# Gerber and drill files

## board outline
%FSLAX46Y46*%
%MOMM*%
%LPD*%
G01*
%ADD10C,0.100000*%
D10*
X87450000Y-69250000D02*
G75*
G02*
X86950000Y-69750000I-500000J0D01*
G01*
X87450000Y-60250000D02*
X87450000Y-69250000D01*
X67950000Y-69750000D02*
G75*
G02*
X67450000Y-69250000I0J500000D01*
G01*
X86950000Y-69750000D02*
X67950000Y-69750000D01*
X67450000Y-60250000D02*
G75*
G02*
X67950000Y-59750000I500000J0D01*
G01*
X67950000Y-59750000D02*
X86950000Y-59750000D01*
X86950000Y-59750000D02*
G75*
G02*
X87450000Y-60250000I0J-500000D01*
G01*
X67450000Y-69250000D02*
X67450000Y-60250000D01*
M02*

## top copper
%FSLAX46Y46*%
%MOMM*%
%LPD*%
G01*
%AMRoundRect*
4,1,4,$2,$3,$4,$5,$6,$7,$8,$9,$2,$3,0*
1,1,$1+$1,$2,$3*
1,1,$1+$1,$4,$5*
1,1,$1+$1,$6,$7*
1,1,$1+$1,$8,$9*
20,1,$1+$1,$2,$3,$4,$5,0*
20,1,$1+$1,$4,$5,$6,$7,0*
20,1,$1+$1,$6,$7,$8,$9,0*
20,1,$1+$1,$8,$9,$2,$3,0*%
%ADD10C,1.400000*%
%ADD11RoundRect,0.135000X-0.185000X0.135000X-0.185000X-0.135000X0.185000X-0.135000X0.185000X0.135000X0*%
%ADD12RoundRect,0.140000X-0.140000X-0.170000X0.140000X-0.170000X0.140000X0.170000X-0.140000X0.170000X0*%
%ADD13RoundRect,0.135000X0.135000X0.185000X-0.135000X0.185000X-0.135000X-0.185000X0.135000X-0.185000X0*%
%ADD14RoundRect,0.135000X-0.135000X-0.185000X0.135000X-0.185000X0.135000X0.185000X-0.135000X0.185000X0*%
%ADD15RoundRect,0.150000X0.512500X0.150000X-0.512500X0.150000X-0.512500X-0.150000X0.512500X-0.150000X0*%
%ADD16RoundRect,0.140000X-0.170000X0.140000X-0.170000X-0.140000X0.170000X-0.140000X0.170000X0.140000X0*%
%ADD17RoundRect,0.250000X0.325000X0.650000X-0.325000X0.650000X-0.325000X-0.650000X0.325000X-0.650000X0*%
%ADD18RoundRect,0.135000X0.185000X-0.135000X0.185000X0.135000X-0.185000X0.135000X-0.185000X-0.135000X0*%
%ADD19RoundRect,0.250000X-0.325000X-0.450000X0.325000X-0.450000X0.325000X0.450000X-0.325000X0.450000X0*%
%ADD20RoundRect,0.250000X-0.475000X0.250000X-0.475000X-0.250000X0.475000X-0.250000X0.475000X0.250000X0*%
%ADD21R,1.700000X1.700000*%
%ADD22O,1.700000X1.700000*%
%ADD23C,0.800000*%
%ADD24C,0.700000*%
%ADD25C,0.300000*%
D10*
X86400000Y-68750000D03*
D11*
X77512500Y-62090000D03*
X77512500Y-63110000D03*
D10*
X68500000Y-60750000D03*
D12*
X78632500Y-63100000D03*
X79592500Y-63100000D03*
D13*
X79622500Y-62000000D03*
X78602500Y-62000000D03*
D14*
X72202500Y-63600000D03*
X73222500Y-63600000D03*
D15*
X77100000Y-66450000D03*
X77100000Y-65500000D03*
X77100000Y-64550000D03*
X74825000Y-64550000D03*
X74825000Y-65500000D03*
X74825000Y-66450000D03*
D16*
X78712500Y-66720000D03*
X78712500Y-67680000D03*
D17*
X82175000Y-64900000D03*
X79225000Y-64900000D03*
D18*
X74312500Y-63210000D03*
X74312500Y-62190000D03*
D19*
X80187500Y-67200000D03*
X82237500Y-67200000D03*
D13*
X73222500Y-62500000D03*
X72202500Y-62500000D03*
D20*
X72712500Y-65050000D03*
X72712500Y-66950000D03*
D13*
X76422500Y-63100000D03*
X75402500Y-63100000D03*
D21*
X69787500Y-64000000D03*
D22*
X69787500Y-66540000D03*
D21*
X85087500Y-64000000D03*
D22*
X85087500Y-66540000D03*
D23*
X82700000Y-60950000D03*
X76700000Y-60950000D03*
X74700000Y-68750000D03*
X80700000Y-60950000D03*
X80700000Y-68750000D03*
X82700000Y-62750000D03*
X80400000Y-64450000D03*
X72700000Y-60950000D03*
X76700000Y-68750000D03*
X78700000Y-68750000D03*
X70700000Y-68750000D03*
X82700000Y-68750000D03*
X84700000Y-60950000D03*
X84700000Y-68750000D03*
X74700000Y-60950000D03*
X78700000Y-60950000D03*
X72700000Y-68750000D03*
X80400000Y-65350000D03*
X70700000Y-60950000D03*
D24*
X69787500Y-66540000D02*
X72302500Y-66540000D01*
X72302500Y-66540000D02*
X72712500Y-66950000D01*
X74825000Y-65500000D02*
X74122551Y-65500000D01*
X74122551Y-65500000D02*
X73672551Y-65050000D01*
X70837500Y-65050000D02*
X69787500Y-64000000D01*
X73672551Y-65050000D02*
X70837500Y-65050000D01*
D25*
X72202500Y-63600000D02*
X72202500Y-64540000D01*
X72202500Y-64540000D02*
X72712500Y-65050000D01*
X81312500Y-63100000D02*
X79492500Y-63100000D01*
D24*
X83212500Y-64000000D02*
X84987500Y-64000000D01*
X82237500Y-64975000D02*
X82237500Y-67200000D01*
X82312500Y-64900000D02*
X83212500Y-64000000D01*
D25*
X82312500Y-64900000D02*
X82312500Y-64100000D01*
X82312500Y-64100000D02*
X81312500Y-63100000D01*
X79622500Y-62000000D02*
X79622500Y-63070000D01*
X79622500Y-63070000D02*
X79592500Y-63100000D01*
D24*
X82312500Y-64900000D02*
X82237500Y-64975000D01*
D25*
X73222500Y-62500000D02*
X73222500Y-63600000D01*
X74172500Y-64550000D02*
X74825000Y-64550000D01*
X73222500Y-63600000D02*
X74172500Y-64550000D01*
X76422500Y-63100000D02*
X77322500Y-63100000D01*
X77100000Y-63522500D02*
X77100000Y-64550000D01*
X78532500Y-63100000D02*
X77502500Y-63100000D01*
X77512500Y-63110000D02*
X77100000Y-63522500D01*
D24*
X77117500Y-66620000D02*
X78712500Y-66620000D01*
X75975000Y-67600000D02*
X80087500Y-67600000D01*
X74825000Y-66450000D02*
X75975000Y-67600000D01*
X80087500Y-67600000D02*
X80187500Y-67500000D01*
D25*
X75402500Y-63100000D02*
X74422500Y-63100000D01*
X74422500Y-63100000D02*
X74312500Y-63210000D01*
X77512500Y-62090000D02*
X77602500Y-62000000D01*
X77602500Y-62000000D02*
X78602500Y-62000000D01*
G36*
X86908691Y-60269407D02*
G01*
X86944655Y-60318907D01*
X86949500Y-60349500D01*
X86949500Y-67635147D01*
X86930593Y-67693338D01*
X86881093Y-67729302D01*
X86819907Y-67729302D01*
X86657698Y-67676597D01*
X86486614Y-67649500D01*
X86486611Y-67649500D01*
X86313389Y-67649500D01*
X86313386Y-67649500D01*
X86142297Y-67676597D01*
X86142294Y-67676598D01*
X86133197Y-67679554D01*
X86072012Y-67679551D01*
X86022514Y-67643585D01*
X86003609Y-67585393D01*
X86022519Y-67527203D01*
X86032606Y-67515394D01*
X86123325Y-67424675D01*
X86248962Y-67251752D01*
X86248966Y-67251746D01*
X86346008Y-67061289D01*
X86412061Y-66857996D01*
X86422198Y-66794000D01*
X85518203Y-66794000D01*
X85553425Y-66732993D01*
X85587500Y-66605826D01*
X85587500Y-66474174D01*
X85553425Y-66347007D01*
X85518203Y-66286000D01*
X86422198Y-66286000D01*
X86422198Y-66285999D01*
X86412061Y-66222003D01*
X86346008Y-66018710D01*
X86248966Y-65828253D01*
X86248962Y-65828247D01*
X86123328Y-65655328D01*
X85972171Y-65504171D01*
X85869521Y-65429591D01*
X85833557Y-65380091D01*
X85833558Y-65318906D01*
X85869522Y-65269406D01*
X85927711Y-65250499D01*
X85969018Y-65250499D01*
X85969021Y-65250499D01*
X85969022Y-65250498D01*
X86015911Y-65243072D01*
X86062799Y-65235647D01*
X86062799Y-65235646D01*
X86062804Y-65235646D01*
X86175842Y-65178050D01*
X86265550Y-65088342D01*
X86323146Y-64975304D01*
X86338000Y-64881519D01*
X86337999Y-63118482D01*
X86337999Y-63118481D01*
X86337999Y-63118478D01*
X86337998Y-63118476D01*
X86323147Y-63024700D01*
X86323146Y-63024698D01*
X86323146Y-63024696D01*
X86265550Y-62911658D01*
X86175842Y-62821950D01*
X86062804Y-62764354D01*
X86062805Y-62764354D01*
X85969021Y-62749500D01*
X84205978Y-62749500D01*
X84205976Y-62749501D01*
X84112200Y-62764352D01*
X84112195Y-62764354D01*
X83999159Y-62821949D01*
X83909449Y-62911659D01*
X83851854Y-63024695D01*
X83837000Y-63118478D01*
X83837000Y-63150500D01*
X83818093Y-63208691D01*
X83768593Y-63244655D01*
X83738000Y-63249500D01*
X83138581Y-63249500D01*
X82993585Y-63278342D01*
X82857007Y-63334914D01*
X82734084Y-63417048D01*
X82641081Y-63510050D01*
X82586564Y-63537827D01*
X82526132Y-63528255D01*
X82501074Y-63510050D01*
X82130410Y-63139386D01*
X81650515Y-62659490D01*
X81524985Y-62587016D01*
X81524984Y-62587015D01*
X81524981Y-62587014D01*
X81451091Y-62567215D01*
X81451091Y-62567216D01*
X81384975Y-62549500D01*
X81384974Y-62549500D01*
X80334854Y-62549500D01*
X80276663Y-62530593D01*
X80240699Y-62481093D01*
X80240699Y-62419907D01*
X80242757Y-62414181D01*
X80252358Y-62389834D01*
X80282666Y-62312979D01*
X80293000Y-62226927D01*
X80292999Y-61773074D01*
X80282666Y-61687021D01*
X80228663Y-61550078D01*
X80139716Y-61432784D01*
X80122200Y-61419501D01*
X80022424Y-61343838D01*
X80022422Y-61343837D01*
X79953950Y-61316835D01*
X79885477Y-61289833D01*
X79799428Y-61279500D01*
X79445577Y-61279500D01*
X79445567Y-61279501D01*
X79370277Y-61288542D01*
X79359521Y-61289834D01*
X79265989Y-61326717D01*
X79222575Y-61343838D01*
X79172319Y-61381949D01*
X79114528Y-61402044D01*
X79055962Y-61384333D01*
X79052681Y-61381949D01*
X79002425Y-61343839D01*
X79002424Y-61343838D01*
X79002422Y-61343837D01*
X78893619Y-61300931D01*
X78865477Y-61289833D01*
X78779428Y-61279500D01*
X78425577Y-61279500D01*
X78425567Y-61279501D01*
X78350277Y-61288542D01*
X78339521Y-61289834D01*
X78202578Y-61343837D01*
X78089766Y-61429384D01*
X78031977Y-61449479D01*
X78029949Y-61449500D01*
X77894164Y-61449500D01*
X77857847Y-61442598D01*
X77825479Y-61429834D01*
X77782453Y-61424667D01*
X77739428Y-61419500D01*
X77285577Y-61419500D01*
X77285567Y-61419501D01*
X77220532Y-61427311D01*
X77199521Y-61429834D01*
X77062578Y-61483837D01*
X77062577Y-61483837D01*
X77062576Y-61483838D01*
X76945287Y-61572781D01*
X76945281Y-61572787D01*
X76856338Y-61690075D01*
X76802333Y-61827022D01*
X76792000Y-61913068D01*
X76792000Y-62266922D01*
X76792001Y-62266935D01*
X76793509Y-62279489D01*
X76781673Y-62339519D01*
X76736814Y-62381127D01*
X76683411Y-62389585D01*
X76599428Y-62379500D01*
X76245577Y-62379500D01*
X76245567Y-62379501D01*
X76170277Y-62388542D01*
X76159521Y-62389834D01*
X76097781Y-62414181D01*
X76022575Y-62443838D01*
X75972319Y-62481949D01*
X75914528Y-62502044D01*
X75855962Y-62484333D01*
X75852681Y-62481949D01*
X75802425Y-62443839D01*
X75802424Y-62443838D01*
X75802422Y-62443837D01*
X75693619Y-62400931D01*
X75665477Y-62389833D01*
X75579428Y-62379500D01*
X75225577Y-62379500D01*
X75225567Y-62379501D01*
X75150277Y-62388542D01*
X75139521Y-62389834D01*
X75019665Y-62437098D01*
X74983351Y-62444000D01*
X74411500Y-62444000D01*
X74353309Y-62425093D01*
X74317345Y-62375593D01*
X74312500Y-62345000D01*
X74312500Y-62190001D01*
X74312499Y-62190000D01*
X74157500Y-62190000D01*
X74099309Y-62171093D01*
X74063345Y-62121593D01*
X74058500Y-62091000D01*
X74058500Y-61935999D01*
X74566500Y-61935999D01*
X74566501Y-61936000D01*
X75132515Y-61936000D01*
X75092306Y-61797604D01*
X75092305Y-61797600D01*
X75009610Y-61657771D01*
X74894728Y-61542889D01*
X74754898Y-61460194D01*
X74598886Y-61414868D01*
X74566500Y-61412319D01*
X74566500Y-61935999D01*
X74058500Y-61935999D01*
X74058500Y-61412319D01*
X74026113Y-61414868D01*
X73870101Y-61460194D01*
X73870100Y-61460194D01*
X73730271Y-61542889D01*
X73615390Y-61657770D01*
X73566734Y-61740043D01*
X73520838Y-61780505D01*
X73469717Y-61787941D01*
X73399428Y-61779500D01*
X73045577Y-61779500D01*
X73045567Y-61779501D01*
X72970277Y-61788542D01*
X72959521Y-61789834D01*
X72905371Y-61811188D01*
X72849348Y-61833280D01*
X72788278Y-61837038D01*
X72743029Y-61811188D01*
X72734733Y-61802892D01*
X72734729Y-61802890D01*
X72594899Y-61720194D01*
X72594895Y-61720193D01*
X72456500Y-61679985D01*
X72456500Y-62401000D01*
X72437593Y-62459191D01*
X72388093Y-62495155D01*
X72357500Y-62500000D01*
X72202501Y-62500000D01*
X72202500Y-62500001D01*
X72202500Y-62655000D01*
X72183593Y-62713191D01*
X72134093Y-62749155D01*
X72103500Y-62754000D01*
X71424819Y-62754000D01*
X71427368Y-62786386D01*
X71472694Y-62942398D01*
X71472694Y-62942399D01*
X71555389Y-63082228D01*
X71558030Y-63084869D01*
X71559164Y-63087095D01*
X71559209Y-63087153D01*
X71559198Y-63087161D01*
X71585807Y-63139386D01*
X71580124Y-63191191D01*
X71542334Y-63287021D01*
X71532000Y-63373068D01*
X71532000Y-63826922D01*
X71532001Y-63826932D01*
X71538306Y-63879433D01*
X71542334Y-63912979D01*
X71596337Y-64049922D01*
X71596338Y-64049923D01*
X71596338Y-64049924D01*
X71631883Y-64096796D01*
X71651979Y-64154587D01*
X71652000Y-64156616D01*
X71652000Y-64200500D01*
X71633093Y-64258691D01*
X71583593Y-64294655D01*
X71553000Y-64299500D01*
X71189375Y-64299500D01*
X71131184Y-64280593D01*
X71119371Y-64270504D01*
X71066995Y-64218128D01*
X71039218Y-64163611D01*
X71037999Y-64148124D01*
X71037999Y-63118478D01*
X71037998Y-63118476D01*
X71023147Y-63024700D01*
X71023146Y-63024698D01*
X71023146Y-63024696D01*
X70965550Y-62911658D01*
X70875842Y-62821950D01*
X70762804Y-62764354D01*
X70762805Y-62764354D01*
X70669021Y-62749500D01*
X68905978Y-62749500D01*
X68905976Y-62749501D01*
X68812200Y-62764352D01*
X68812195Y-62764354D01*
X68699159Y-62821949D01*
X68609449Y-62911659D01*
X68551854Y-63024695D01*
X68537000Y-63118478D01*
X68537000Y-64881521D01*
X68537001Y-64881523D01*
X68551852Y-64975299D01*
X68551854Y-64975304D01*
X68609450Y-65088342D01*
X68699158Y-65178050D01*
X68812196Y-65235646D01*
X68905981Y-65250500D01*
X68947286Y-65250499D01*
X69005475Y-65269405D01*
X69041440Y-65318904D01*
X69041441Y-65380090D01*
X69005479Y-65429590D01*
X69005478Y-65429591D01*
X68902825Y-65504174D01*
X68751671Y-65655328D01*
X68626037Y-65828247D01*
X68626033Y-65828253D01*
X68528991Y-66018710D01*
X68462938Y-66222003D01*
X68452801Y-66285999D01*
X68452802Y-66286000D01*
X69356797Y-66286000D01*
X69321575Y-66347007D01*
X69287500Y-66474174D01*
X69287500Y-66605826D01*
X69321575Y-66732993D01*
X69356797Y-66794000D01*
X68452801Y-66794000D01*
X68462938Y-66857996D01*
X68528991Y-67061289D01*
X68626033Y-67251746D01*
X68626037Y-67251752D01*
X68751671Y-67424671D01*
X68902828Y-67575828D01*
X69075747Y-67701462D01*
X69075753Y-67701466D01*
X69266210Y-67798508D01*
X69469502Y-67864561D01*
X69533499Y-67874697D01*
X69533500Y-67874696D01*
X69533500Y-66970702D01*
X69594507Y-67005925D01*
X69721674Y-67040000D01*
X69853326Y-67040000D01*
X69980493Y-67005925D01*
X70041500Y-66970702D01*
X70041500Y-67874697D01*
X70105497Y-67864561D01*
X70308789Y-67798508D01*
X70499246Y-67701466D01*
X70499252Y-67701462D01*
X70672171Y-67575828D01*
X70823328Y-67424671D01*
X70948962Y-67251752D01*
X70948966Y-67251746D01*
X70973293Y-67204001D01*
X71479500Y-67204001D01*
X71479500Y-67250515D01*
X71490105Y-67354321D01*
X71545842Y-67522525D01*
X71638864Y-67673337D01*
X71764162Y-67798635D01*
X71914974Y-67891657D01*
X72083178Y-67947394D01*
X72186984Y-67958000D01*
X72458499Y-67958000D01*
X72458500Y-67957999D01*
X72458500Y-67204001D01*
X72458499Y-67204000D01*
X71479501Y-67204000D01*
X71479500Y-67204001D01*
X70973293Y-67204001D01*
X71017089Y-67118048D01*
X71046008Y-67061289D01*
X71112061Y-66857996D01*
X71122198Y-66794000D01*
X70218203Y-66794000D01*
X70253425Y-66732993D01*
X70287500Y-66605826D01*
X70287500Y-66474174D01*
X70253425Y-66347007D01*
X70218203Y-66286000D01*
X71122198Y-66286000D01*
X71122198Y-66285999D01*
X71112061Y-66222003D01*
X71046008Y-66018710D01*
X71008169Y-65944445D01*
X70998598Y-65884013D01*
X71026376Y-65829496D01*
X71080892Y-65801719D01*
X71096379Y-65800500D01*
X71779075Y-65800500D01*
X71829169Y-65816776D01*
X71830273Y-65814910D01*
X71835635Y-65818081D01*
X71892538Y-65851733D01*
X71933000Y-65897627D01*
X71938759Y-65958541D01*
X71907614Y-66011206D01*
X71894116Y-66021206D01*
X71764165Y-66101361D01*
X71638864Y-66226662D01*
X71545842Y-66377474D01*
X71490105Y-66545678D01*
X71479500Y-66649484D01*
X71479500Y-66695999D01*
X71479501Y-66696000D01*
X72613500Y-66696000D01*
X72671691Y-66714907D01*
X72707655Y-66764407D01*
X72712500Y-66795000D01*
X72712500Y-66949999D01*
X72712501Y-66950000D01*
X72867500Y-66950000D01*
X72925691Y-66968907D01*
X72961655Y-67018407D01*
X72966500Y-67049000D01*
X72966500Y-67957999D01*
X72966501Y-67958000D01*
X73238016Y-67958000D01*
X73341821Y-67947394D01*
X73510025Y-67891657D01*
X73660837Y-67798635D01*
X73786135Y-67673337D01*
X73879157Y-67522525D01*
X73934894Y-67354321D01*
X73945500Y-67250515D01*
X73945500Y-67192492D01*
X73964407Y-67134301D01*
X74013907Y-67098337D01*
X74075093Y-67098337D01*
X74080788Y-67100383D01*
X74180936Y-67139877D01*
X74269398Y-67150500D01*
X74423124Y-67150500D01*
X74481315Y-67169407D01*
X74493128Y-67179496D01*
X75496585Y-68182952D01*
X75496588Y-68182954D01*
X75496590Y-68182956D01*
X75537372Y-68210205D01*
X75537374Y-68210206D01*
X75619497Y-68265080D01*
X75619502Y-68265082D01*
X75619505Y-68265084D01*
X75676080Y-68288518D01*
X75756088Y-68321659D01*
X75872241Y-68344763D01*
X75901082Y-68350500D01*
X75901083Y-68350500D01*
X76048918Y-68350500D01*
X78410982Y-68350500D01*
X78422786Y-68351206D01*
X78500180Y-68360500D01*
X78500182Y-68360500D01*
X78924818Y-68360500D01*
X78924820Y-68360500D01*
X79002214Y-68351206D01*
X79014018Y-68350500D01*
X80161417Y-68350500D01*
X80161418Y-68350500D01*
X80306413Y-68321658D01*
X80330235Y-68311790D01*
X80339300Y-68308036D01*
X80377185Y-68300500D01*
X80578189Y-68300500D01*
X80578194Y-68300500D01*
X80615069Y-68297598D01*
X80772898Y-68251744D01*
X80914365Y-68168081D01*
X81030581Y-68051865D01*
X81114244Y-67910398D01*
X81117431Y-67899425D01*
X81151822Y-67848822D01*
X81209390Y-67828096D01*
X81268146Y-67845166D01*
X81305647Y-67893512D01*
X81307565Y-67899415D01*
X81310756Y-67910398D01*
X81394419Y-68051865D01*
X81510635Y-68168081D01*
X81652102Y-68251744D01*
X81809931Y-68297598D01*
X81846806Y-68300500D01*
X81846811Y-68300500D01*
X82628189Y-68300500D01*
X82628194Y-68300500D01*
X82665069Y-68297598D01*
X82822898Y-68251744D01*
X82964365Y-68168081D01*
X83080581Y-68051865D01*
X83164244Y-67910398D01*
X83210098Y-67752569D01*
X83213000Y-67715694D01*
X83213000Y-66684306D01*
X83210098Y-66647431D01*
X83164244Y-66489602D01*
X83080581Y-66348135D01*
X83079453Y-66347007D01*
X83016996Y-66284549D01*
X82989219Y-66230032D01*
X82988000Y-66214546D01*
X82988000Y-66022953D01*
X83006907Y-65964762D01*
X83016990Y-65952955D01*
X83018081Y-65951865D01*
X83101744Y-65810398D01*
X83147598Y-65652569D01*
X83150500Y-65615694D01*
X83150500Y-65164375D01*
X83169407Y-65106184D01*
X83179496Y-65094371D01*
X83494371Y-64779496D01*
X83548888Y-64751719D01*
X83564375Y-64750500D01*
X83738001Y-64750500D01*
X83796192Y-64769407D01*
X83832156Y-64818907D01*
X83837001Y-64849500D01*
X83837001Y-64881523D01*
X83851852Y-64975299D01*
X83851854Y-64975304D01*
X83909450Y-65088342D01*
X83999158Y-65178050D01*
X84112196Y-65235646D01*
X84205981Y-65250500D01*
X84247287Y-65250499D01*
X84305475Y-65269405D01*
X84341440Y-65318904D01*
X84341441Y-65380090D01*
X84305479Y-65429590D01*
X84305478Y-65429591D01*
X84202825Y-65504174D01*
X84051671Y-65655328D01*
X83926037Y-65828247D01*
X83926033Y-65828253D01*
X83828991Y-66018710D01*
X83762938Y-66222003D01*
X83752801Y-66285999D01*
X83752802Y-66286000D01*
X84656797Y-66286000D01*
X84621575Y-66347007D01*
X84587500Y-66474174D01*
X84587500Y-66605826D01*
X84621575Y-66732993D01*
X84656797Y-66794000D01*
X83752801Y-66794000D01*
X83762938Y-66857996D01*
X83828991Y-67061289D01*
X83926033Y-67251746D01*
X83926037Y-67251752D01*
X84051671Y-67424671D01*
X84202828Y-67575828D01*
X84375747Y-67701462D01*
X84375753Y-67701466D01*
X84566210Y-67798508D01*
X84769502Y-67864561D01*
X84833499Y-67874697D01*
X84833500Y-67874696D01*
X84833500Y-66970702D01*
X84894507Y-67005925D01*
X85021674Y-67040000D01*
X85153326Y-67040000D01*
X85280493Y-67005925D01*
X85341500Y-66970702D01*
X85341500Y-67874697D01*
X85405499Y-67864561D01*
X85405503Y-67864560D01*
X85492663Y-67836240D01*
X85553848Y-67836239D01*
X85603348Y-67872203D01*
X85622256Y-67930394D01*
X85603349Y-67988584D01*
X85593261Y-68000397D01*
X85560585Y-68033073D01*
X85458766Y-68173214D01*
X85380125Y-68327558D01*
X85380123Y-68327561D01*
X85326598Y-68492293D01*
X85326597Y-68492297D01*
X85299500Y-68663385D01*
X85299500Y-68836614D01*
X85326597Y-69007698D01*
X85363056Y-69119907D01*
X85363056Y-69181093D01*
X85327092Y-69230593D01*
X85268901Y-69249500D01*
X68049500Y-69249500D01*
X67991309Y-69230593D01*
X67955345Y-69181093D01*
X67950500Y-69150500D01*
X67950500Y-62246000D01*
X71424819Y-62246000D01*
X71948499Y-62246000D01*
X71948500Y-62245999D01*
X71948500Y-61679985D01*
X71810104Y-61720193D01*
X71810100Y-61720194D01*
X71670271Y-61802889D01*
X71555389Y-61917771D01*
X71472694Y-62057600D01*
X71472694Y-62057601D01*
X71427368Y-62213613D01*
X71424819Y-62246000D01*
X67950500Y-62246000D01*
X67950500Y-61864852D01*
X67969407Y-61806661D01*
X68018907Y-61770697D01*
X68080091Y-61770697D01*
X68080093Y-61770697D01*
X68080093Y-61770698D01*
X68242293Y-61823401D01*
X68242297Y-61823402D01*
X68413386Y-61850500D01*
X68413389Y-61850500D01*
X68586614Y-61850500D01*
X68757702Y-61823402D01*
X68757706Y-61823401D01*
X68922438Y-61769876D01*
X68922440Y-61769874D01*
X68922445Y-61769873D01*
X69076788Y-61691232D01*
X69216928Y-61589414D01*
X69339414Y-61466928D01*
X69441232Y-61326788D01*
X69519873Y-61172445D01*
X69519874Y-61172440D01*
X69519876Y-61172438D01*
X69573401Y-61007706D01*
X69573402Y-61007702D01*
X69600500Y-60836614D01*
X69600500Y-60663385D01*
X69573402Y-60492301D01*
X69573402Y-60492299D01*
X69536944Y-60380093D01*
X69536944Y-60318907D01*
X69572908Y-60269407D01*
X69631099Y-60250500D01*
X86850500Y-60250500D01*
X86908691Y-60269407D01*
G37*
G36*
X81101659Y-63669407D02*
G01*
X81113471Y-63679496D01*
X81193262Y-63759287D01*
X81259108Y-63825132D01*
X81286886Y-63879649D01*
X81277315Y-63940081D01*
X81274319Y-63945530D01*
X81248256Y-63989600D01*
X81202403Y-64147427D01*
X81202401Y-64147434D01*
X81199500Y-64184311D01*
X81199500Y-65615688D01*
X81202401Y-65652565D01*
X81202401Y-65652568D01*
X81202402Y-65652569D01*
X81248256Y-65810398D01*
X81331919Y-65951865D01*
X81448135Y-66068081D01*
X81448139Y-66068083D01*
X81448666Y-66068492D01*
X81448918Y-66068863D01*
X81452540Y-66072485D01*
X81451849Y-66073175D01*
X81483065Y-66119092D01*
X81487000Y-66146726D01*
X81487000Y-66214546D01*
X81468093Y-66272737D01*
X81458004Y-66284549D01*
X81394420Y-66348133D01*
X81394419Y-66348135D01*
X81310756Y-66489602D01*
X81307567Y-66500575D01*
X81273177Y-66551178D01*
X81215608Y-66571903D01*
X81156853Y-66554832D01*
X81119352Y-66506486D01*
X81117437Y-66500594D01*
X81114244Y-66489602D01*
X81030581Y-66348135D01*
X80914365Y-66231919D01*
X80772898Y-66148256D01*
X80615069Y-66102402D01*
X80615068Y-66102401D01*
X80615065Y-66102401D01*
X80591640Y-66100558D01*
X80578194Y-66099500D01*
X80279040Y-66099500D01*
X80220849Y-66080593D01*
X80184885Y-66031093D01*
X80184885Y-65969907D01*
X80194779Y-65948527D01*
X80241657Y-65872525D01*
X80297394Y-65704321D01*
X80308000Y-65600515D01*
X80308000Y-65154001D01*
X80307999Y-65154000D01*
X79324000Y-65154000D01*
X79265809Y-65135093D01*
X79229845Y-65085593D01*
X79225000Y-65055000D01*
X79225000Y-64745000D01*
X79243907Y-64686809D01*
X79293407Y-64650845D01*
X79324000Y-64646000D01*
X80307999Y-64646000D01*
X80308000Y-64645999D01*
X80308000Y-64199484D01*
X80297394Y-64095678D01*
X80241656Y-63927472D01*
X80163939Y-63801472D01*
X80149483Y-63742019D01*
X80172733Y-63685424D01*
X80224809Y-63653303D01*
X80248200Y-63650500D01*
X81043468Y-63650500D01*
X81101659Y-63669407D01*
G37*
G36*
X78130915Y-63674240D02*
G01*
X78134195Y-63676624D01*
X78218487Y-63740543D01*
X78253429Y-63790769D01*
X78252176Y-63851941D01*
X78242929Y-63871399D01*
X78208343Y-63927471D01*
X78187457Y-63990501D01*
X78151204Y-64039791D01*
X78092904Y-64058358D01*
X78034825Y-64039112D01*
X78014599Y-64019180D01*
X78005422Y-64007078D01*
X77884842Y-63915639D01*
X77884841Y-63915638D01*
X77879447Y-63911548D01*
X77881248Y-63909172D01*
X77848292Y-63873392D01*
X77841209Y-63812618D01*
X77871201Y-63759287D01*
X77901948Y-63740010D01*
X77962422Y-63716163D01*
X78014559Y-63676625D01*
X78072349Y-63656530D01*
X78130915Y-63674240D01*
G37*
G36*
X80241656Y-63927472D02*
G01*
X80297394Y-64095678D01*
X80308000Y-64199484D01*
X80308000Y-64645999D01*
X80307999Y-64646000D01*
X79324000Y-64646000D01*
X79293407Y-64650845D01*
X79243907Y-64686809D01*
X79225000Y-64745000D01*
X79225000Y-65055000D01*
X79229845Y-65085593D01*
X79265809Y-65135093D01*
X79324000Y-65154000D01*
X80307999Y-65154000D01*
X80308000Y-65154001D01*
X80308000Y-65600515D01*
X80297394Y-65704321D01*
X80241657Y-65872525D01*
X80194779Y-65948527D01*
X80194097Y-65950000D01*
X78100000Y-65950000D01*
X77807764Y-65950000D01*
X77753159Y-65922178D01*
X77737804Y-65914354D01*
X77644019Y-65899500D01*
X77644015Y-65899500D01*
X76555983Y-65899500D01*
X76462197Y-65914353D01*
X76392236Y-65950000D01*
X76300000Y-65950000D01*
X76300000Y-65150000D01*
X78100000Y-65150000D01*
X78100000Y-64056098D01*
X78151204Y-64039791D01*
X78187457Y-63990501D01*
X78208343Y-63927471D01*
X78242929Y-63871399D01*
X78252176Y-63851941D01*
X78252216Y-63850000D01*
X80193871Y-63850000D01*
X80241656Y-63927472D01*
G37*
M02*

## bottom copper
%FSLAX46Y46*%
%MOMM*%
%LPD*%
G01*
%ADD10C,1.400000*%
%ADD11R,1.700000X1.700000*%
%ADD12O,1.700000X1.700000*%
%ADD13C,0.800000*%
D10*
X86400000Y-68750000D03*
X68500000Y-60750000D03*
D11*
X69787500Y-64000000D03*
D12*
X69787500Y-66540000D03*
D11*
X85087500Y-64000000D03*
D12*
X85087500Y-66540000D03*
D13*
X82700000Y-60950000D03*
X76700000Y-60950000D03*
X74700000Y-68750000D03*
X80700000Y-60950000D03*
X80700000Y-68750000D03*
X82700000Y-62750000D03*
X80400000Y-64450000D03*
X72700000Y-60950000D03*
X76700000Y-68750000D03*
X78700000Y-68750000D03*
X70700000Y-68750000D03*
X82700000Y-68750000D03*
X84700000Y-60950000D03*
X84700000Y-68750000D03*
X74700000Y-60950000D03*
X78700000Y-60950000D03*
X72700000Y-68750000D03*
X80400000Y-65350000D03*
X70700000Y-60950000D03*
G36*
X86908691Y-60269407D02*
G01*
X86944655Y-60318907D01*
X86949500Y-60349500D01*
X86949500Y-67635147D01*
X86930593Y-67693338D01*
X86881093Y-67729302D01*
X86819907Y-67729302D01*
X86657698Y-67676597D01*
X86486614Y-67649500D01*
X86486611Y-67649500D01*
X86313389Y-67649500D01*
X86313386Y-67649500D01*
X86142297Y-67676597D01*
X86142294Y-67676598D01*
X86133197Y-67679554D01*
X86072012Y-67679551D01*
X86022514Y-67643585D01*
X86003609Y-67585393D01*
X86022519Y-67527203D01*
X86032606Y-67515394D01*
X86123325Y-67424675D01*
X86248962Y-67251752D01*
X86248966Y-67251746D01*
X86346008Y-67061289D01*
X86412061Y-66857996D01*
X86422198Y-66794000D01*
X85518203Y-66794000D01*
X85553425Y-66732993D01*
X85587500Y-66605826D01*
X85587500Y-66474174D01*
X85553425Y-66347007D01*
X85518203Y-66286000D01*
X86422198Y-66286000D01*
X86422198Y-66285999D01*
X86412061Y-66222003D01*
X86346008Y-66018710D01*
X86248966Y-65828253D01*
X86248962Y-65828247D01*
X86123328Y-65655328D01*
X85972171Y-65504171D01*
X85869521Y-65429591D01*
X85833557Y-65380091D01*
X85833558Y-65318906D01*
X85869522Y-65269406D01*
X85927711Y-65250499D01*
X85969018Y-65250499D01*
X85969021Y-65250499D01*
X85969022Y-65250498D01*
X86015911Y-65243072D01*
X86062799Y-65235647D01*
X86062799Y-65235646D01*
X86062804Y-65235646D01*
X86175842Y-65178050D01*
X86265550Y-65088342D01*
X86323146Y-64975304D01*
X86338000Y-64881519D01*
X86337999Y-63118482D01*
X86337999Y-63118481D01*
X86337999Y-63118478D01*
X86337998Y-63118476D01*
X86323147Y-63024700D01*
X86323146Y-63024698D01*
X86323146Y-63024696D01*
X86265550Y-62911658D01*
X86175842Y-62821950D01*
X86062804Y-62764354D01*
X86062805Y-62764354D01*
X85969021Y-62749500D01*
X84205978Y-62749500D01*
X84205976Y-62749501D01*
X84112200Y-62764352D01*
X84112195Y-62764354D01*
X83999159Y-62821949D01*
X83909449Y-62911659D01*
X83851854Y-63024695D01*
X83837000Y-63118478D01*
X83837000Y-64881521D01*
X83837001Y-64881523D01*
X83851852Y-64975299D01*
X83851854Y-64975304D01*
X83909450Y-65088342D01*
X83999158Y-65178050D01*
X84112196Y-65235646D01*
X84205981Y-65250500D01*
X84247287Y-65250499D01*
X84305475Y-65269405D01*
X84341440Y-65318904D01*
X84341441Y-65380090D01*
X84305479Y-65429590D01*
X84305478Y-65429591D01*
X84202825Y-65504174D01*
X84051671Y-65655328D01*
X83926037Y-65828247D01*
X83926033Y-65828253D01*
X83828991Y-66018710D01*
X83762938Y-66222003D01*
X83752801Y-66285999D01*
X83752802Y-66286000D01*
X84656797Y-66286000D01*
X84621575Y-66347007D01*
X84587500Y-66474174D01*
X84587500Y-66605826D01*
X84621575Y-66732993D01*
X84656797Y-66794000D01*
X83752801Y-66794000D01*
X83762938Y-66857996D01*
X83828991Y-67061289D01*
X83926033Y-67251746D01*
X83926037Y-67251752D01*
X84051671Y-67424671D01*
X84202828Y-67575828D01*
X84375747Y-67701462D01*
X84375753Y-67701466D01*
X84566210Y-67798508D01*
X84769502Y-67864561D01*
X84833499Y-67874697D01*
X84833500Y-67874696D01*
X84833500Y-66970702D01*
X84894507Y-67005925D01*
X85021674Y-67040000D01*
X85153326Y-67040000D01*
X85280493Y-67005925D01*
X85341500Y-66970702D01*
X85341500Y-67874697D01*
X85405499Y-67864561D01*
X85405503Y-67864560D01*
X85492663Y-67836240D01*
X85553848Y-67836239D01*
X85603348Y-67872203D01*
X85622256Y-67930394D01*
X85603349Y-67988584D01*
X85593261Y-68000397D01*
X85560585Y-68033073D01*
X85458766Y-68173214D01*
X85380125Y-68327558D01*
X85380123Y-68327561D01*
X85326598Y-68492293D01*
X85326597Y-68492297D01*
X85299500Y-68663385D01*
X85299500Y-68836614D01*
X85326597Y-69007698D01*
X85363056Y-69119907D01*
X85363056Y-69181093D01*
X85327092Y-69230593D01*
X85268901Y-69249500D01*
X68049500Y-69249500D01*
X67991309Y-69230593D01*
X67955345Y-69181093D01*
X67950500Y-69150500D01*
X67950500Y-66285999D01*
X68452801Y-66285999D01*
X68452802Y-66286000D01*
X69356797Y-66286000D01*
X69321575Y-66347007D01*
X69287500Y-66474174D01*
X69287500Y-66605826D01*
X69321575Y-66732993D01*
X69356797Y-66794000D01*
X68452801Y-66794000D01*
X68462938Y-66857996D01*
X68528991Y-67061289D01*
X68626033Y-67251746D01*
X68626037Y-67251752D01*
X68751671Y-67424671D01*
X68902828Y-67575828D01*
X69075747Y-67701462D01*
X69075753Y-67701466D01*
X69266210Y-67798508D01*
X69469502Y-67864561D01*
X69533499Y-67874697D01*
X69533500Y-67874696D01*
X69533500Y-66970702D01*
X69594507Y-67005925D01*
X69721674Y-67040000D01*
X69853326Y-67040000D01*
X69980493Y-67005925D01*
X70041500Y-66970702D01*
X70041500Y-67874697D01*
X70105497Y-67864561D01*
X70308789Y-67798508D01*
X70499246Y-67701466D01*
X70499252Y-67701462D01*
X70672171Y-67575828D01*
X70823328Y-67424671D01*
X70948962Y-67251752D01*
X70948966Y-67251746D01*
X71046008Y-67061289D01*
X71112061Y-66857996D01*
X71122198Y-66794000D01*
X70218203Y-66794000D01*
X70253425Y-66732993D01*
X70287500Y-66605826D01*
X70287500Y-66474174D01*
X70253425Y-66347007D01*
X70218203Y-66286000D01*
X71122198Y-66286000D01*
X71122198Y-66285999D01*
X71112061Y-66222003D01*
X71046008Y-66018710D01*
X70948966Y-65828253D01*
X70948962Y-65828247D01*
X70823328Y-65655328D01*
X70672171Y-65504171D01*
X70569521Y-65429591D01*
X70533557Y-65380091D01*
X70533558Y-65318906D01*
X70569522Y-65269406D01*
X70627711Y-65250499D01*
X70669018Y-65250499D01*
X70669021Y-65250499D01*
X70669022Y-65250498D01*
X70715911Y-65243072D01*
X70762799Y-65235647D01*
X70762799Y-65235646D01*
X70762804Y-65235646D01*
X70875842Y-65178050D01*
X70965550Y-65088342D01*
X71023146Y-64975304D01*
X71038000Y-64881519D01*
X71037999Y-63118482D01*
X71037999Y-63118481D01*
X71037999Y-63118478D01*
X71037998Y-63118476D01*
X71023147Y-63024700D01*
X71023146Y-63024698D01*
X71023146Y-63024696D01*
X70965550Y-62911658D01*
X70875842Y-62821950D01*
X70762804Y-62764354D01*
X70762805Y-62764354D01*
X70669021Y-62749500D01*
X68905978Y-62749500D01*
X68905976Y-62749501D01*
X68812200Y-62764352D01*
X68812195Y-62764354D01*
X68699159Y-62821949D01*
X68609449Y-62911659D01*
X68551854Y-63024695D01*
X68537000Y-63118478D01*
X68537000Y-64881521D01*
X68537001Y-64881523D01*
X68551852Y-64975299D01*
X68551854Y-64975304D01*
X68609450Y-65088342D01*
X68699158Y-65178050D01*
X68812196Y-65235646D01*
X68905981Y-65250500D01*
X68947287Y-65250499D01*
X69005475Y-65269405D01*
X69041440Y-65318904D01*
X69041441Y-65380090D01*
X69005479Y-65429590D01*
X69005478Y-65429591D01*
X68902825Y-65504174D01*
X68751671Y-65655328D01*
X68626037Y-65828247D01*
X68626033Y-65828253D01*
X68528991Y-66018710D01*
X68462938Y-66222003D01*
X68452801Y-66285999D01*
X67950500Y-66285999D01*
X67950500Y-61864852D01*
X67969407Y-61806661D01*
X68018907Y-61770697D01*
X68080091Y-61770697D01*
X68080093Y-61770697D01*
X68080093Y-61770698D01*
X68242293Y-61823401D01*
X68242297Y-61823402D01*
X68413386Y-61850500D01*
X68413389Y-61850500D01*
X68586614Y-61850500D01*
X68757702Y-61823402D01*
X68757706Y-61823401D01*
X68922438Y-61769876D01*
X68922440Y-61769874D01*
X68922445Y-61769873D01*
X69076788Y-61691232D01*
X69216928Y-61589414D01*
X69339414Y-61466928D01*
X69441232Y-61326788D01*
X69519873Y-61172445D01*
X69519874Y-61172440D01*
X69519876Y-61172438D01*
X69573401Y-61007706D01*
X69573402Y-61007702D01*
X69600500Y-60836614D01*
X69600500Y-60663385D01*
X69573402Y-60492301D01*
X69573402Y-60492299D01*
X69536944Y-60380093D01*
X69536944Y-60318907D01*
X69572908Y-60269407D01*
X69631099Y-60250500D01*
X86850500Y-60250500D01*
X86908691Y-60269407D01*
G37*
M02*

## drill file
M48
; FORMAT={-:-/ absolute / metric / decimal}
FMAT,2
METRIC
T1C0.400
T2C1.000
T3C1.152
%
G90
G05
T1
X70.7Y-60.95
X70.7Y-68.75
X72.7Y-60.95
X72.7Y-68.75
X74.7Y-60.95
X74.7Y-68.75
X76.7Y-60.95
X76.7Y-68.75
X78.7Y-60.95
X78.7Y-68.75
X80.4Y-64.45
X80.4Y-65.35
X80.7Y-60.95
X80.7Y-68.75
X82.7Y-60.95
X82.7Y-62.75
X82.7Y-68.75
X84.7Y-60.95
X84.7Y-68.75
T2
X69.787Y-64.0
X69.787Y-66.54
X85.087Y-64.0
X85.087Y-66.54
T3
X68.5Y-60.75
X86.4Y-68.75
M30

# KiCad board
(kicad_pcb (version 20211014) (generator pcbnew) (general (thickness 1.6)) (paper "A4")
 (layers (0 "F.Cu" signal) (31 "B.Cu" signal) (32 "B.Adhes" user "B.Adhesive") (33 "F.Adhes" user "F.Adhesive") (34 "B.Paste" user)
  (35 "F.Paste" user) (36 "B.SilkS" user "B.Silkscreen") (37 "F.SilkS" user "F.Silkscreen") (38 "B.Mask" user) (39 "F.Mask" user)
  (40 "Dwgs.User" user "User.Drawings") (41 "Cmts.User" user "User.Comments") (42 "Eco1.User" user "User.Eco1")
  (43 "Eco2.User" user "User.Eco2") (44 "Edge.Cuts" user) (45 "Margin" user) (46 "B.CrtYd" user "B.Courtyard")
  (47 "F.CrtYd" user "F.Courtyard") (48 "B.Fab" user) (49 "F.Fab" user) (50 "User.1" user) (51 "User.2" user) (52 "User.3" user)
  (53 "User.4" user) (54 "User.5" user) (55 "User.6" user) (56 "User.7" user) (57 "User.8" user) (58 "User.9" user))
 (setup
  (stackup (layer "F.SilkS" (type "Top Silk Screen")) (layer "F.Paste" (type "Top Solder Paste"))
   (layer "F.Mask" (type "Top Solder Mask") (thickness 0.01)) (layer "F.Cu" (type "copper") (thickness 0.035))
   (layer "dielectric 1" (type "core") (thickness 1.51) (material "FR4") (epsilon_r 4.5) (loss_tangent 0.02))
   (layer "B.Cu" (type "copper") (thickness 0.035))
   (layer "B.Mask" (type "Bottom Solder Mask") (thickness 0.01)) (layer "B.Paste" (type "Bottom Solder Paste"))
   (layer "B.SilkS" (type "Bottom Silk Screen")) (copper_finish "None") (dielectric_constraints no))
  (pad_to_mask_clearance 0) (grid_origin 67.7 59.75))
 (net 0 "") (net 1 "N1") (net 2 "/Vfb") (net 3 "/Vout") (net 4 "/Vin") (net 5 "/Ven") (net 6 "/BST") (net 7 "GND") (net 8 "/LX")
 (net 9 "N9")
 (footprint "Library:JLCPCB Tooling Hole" (layer "F.Cu") (at 86.4 68.75)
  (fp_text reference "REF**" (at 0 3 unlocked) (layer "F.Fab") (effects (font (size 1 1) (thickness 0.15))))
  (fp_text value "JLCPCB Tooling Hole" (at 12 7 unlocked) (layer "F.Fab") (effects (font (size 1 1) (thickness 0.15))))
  (pad "" np_thru_hole circle (at 0 0) (size 1.4 1.4) (drill 1.152) (layers F&B.Cu *.Mask)))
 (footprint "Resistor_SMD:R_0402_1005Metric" (layer "F.Cu") (at 77.5125 62.6 -90)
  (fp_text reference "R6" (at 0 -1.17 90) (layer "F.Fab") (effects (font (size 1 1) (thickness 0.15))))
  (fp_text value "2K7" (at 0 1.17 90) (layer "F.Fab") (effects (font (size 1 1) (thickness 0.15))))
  (pad "1" smd roundrect (at -0.51 0 270) (size 0.54 0.64) (layers "F.Cu" "F.Paste" "F.Mask") (roundrect_rratio 0.25) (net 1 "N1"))
  (pad "2" smd roundrect (at 0.51 0 270) (size 0.54 0.64) (layers "F.Cu" "F.Paste" "F.Mask") (roundrect_rratio 0.25) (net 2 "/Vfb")))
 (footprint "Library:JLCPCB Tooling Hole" (layer "F.Cu") (at 68.5 60.75)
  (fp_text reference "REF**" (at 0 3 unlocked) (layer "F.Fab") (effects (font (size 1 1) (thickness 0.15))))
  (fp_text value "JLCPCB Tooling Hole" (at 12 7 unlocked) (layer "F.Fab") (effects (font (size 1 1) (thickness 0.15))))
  (pad "" np_thru_hole circle (at 0 0) (size 1.4 1.4) (drill 1.152) (layers F&B.Cu *.Mask)))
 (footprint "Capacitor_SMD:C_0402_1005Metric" (layer "F.Cu") (at 79.1125 63.1)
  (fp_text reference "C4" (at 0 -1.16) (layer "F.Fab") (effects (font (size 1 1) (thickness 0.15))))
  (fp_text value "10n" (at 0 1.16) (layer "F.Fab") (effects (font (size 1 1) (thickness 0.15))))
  (pad "1" smd roundrect (at -0.48 0) (size 0.56 0.62) (layers "F.Cu" "F.Paste" "F.Mask") (roundrect_rratio 0.25) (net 2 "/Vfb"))
  (pad "2" smd roundrect (at 0.48 0) (size 0.56 0.62) (layers "F.Cu" "F.Paste" "F.Mask") (roundrect_rratio 0.25) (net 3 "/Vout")))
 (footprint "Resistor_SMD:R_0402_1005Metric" (layer "F.Cu") (at 79.1125 62 180)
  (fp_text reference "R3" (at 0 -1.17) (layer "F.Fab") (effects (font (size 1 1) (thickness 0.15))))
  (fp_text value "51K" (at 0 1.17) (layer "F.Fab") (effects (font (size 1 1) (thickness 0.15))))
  (pad "1" smd roundrect (at -0.51 0 180) (size 0.54 0.64) (layers "F.Cu" "F.Paste" "F.Mask") (roundrect_rratio 0.25) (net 3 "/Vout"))
  (pad "2" smd roundrect (at 0.51 0 180) (size 0.54 0.64) (layers "F.Cu" "F.Paste" "F.Mask") (roundrect_rratio 0.25) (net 1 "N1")))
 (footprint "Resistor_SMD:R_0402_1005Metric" (layer "F.Cu") (at 72.7125 63.6)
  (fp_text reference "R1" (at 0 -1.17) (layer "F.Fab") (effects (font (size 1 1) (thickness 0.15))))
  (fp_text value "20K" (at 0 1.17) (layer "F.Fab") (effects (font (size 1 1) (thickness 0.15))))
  (pad "1" smd roundrect (at -0.51 0) (size 0.54 0.64) (layers "F.Cu" "F.Paste" "F.Mask") (roundrect_rratio 0.25) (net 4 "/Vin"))
  (pad "2" smd roundrect (at 0.51 0) (size 0.54 0.64) (layers "F.Cu" "F.Paste" "F.Mask") (roundrect_rratio 0.25) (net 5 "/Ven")))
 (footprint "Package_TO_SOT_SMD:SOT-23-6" (layer "F.Cu") (at 75.9625 65.5 180)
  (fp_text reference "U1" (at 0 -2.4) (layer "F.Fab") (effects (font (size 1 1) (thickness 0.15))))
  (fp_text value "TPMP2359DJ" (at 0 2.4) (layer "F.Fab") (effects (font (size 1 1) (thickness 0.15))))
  (pad "1" smd roundrect (at -1.1375 -0.95 180) (size 1.325 0.6) (layers "F.Cu" "F.Paste" "F.Mask") (roundrect_rratio 0.25) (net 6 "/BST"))
  (pad "2" smd roundrect (at -1.1375 0 180) (size 1.325 0.6) (layers "F.Cu" "F.Paste" "F.Mask") (roundrect_rratio 0.25) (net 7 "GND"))
  (pad "3" smd roundrect (at -1.1375 0.95 180) (size 1.325 0.6) (layers "F.Cu" "F.Paste" "F.Mask") (roundrect_rratio 0.25) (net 2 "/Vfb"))
  (pad "4" smd roundrect (at 1.1375 0.95 180) (size 1.325 0.6) (layers "F.Cu" "F.Paste" "F.Mask") (roundrect_rratio 0.25) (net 5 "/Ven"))
  (pad "5" smd roundrect (at 1.1375 0 180) (size 1.325 0.6) (layers "F.Cu" "F.Paste" "F.Mask") (roundrect_rratio 0.25) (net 4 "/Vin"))
  (pad "6" smd roundrect (at 1.1375 -0.95 180) (size 1.325 0.6) (layers "F.Cu" "F.Paste" "F.Mask") (roundrect_rratio 0.25) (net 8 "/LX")))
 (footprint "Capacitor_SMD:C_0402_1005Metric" (layer "F.Cu") (at 78.7125 67.2 -90)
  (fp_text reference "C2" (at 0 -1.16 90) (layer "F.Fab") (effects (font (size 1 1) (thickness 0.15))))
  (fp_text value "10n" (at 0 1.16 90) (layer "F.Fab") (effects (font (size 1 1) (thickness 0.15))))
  (pad "1" smd roundrect (at -0.48 0 270) (size 0.56 0.62) (layers "F.Cu" "F.Paste" "F.Mask") (roundrect_rratio 0.25) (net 6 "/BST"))
  (pad "2" smd roundrect (at 0.48 0 270) (size 0.56 0.62) (layers "F.Cu" "F.Paste" "F.Mask") (roundrect_rratio 0.25) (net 8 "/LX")))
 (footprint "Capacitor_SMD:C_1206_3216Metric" (layer "F.Cu") (at 80.7 64.9 180)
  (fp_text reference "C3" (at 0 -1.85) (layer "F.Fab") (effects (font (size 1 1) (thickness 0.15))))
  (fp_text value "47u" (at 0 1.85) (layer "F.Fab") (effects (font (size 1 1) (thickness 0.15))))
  (pad "1" smd roundrect (at -1.475 0 180) (size 1.15 1.8) (layers "F.Cu" "F.Paste" "F.Mask") (roundrect_rratio 0.2173913043)
   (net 3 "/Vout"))
  (pad "2" smd roundrect (at 1.475 0 180) (size 1.15 1.8) (layers "F.Cu" "F.Paste" "F.Mask") (roundrect_rratio 0.2173913043) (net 7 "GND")))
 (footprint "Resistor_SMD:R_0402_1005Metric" (layer "F.Cu") (at 74.3125 62.7 90)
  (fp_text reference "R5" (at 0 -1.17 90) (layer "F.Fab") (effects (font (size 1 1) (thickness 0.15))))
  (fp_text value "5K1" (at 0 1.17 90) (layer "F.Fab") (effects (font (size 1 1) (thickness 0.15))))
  (pad "1" smd roundrect (at -0.51 0 90) (size 0.54 0.64) (layers "F.Cu" "F.Paste" "F.Mask") (roundrect_rratio 0.25) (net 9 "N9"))
  (pad "2" smd roundrect (at 0.51 0 90) (size 0.54 0.64) (layers "F.Cu" "F.Paste" "F.Mask") (roundrect_rratio 0.25) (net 7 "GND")))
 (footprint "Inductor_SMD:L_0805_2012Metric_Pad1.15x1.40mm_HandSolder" (layer "F.Cu") (at 81.2125 67.2)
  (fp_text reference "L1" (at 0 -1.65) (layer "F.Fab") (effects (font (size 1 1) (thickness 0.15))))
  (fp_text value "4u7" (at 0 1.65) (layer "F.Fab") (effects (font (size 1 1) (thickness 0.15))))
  (pad "1" smd roundrect (at -1.025 0) (size 1.15 1.4) (layers "F.Cu" "F.Paste" "F.Mask") (roundrect_rratio 0.2173913043) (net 8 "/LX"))
  (pad "2" smd roundrect (at 1.025 0) (size 1.15 1.4) (layers "F.Cu" "F.Paste" "F.Mask") (roundrect_rratio 0.2173913043) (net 3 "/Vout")))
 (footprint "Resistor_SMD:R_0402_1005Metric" (layer "F.Cu") (at 72.7125 62.5 180)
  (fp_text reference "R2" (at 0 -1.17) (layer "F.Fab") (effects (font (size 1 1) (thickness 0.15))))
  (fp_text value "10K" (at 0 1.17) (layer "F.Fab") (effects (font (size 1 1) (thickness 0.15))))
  (pad "1" smd roundrect (at -0.51 0 180) (size 0.54 0.64) (layers "F.Cu" "F.Paste" "F.Mask") (roundrect_rratio 0.25) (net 5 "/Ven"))
  (pad "2" smd roundrect (at 0.51 0 180) (size 0.54 0.64) (layers "F.Cu" "F.Paste" "F.Mask") (roundrect_rratio 0.25) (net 7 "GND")))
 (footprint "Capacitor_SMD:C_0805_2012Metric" (layer "F.Cu") (at 72.7125 66 -90)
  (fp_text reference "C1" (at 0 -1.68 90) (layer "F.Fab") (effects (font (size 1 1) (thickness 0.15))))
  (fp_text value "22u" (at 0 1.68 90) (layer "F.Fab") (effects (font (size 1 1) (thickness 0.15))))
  (pad "1" smd roundrect (at -0.95 0 270) (size 1 1.45) (layers "F.Cu" "F.Paste" "F.Mask") (roundrect_rratio 0.25) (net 4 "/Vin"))
  (pad "2" smd roundrect (at 0.95 0 270) (size 1 1.45) (layers "F.Cu" "F.Paste" "F.Mask") (roundrect_rratio 0.25) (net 7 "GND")))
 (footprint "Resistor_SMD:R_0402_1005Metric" (layer "F.Cu") (at 75.9125 63.1 180)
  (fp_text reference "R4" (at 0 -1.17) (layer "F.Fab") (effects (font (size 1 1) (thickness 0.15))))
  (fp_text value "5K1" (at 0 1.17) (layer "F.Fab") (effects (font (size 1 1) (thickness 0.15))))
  (pad "1" smd roundrect (at -0.51 0 180) (size 0.54 0.64) (layers "F.Cu" "F.Paste" "F.Mask") (roundrect_rratio 0.25) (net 2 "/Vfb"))
  (pad "2" smd roundrect (at 0.51 0 180) (size 0.54 0.64) (layers "F.Cu" "F.Paste" "F.Mask") (roundrect_rratio 0.25) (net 9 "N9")))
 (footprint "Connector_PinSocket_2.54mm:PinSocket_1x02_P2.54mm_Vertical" (layer "B.Cu") (at 69.7875 64 180)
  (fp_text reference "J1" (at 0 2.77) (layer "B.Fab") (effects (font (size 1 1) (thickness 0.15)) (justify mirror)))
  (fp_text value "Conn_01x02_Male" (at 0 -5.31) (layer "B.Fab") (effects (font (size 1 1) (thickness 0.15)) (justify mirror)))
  (pad "1" thru_hole rect (at 0 0 180) (size 1.7 1.7) (drill 1) (layers *.Cu *.Mask) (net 4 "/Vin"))
  (pad "2" thru_hole oval (at 0 -2.54 180) (size 1.7 1.7) (drill 1) (layers *.Cu *.Mask) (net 7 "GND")))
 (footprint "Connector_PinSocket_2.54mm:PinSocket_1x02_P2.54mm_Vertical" (layer "B.Cu") (at 85.0875 64 180)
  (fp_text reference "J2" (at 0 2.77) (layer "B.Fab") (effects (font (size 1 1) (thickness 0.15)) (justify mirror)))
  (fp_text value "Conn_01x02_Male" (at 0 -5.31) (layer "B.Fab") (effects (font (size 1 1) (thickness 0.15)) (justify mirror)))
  (pad "1" thru_hole rect (at 0 0 180) (size 1.7 1.7) (drill 1) (layers *.Cu *.Mask) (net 3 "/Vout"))
  (pad "2" thru_hole oval (at 0 -2.54 180) (size 1.7 1.7) (drill 1) (layers *.Cu *.Mask) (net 7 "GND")))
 (gr_arc (start 87.45 69.25) (mid 87.303553 69.603553) (end 86.95 69.75) (layer "Edge.Cuts") (width 0.1))
 (gr_line (start 87.45 60.25) (end 87.45 69.25) (layer "Edge.Cuts") (width 0.1))
 (gr_arc (start 67.95 69.75) (mid 67.596447 69.603553) (end 67.45 69.25) (layer "Edge.Cuts") (width 0.1))
 (gr_line (start 86.95 69.75) (end 67.95 69.75) (layer "Edge.Cuts") (width 0.1))
 (gr_arc (start 67.45 60.25) (mid 67.596447 59.896447) (end 67.95 59.75) (layer "Edge.Cuts") (width 0.1))
 (gr_line (start 67.95 59.75) (end 86.95 59.75) (layer "Edge.Cuts") (width 0.1))
 (gr_arc (start 86.95 59.75) (mid 87.303553 59.896447) (end 87.45 60.25) (layer "Edge.Cuts") (width 0.1))
 (gr_line (start 67.45 69.25) (end 67.45 60.25) (layer "Edge.Cuts") (width 0.1))
 (segment (start 69.7875 66.54) (end 72.3025 66.54) (width 0.7) (layer "F.Cu") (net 7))
 (segment (start 72.3025 66.54) (end 72.7125 66.95) (width 0.7) (layer "F.Cu") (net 7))
 (via (at 82.7 60.95) (size 0.8) (drill 0.4) (layers "F.Cu" "B.Cu") (free) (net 7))
 (via (at 76.7 60.95) (size 0.8) (drill 0.4) (layers "F.Cu" "B.Cu") (free) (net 7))
 (via (at 74.7 68.75) (size 0.8) (drill 0.4) (layers "F.Cu" "B.Cu") (free) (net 7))
 (via (at 80.7 60.95) (size 0.8) (drill 0.4) (layers "F.Cu" "B.Cu") (free) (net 7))
 (via (at 80.7 68.75) (size 0.8) (drill 0.4) (layers "F.Cu" "B.Cu") (free) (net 7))
 (via (at 82.7 62.75) (size 0.8) (drill 0.4) (layers "F.Cu" "B.Cu") (free) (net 7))
 (via (at 80.4 64.45) (size 0.8) (drill 0.4) (layers "F.Cu" "B.Cu") (free) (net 7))
 (via (at 72.7 60.95) (size 0.8) (drill 0.4) (layers "F.Cu" "B.Cu") (free) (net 7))
 (via (at 76.7 68.75) (size 0.8) (drill 0.4) (layers "F.Cu" "B.Cu") (free) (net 7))
 (via (at 78.7 68.75) (size 0.8) (drill 0.4) (layers "F.Cu" "B.Cu") (free) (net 7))
 (via (at 70.7 68.75) (size 0.8) (drill 0.4) (layers "F.Cu" "B.Cu") (free) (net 7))
 (via (at 82.7 68.75) (size 0.8) (drill 0.4) (layers "F.Cu" "B.Cu") (free) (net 7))
 (via (at 84.7 60.95) (size 0.8) (drill 0.4) (layers "F.Cu" "B.Cu") (free) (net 7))
 (via (at 84.7 68.75) (size 0.8) (drill 0.4) (layers "F.Cu" "B.Cu") (free) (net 7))
 (via (at 74.7 60.95) (size 0.8) (drill 0.4) (layers "F.Cu" "B.Cu") (free) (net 7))
 (via (at 78.7 60.95) (size 0.8) (drill 0.4) (layers "F.Cu" "B.Cu") (free) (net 7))
 (via (at 72.7 68.75) (size 0.8) (drill 0.4) (layers "F.Cu" "B.Cu") (free) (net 7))
 (via (at 80.4 65.35) (size 0.8) (drill 0.4) (layers "F.Cu" "B.Cu") (free) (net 7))
 (via (at 70.7 60.95) (size 0.8) (drill 0.4) (layers "F.Cu" "B.Cu") (free) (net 7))
 (segment (start 74.825 65.5) (end 74.122551 65.5) (width 0.7) (layer "F.Cu") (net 4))
 (segment (start 74.122551 65.5) (end 73.672551 65.05) (width 0.7) (layer "F.Cu") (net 4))
 (segment (start 70.8375 65.05) (end 69.7875 64) (width 0.7) (layer "F.Cu") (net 4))
 (segment (start 73.672551 65.05) (end 70.8375 65.05) (width 0.7) (layer "F.Cu") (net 4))
 (segment (start 72.2025 63.6) (end 72.2025 64.54) (width 0.3) (layer "F.Cu") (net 4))
 (segment (start 72.2025 64.54) (end 72.7125 65.05) (width 0.3) (layer "F.Cu") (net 4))
 (segment (start 81.3125 63.1) (end 79.4925 63.1) (width 0.3) (layer "F.Cu") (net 3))
 (segment (start 83.2125 64) (end 84.9875 64) (width 0.7) (layer "F.Cu") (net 3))
 (segment (start 82.2375 64.975) (end 82.2375 67.2) (width 0.7) (layer "F.Cu") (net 3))
 (segment (start 82.3125 64.9) (end 83.2125 64) (width 0.7) (layer "F.Cu") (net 3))
 (segment (start 82.3125 64.9) (end 82.3125 64.1) (width 0.3) (layer "F.Cu") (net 3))
 (segment (start 82.3125 64.1) (end 81.3125 63.1) (width 0.3) (layer "F.Cu") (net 3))
 (segment (start 79.6225 62) (end 79.6225 63.07) (width 0.3) (layer "F.Cu") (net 3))
 (segment (start 79.6225 63.07) (end 79.5925 63.1) (width 0.3) (layer "F.Cu") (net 3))
 (segment (start 82.3125 64.9) (end 82.2375 64.975) (width 0.7) (layer "F.Cu") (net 3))
 (segment (start 73.2225 62.5) (end 73.2225 63.6) (width 0.3) (layer "F.Cu") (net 5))
 (segment (start 74.1725 64.55) (end 74.825 64.55) (width 0.3) (layer "F.Cu") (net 5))
 (segment (start 73.2225 63.6) (end 74.1725 64.55) (width 0.3) (layer "F.Cu") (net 5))
 (segment (start 76.4225 63.1) (end 77.3225 63.1) (width 0.3) (layer "F.Cu") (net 2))
 (segment (start 77.1 63.5225) (end 77.1 64.55) (width 0.3) (layer "F.Cu") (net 2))
 (segment (start 78.5325 63.1) (end 77.5025 63.1) (width 0.3) (layer "F.Cu") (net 2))
 (segment (start 77.5125 63.11) (end 77.1 63.5225) (width 0.3) (layer "F.Cu") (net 2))
 (segment (start 77.1175 66.62) (end 78.7125 66.62) (width 0.7) (layer "F.Cu") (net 6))
 (segment (start 75.975 67.6) (end 80.0875 67.6) (width 0.7) (layer "F.Cu") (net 8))
 (segment (start 74.825 66.45) (end 75.975 67.6) (width 0.7) (layer "F.Cu") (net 8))
 (segment (start 80.0875 67.6) (end 80.1875 67.5) (width 0.7) (layer "F.Cu") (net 8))
 (segment (start 75.4025 63.1) (end 74.4225 63.1) (width 0.3) (layer "F.Cu") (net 9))
 (segment (start 74.4225 63.1) (end 74.3125 63.21) (width 0.3) (layer "F.Cu") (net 9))
 (segment (start 77.5125 62.09) (end 77.6025 62) (width 0.3) (layer "F.Cu") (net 1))
 (segment (start 77.6025 62) (end 78.6025 62) (width 0.3) (layer "F.Cu") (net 1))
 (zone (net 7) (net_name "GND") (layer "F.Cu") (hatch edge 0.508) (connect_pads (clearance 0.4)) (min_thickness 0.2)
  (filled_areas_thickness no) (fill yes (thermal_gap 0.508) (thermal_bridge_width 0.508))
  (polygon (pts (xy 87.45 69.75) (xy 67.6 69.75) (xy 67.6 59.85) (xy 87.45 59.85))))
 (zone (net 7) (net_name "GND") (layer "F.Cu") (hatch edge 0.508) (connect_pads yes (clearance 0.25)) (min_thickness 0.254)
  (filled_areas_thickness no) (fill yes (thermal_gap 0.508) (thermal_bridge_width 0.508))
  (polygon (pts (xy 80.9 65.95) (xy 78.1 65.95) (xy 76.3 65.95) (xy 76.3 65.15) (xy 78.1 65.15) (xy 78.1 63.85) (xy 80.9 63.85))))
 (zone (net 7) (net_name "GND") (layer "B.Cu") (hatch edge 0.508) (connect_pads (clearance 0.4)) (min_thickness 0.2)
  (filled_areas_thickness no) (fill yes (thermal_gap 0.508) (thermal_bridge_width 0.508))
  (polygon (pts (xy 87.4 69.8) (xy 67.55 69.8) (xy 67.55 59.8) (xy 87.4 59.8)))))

